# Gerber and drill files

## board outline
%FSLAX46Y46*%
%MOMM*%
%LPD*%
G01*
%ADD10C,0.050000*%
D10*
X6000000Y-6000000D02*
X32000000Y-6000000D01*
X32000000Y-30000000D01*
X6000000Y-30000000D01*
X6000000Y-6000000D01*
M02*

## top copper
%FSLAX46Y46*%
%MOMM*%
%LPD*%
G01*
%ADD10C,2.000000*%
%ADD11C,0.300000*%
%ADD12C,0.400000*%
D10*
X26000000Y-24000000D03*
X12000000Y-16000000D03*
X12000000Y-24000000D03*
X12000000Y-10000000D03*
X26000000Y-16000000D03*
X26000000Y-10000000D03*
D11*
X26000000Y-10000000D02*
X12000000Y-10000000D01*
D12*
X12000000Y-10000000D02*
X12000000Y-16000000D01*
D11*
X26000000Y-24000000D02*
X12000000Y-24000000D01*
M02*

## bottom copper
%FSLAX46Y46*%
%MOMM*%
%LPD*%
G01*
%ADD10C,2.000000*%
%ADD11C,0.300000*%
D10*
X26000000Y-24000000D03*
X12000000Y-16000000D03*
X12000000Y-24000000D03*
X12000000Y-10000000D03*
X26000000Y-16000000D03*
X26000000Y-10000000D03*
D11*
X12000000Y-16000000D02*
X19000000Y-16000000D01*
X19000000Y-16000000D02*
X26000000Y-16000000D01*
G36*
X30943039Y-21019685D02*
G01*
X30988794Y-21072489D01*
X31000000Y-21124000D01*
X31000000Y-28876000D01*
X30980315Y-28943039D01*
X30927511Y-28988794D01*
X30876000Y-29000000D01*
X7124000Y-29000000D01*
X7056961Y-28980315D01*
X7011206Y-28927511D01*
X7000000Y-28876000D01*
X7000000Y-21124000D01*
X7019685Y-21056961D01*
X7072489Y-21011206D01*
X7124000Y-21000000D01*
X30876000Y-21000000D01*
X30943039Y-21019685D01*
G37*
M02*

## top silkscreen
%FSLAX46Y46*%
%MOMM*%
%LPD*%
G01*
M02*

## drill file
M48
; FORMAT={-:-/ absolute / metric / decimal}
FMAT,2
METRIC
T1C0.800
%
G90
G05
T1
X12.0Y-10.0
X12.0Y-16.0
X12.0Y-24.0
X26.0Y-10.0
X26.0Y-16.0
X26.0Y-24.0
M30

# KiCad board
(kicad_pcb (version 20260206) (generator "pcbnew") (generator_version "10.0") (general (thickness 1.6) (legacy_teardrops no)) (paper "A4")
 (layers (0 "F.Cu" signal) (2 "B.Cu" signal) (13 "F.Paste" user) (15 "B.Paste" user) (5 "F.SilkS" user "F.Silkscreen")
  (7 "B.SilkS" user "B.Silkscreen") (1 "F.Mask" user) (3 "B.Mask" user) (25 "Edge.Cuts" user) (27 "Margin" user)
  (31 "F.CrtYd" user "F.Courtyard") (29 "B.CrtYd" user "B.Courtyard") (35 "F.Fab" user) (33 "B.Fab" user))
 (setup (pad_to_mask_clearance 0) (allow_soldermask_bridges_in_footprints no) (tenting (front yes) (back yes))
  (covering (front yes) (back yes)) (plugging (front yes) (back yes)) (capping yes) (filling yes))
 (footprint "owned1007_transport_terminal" (layer "F.Cu") (at 26 24)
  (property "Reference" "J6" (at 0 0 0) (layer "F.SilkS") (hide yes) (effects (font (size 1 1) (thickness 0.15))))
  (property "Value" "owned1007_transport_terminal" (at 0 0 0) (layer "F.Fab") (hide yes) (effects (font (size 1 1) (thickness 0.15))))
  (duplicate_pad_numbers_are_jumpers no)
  (pad "1" thru_hole circle (at 0 0) (size 2 2) (drill 0.8) (layers "*.Cu" "*.Mask") (remove_unused_layers no) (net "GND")))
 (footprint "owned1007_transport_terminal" (layer "F.Cu") (at 12 16)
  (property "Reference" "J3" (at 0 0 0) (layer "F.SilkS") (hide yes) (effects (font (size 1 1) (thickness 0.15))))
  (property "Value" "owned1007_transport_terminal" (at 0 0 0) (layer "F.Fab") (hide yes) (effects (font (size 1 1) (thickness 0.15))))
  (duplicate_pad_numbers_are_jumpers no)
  (pad "1" thru_hole circle (at 0 0) (size 2 2) (drill 0.8) (layers "*.Cu" "*.Mask") (remove_unused_layers no) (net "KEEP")))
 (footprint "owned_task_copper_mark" (layer "F.Cu") (at 10 28)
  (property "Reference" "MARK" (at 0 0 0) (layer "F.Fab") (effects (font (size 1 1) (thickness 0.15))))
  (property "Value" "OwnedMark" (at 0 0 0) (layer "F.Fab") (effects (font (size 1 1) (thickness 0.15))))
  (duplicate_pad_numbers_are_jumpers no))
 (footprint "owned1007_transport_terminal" (layer "F.Cu") (at 12 24)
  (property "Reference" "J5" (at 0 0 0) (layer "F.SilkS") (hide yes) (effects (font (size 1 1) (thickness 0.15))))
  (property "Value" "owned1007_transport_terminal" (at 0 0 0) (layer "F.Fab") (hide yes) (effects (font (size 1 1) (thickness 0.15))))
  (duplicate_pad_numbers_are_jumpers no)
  (pad "1" thru_hole circle (at 0 0) (size 2 2) (drill 0.8) (layers "*.Cu" "*.Mask") (remove_unused_layers no) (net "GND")))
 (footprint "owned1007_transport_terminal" (layer "F.Cu") (at 12 10)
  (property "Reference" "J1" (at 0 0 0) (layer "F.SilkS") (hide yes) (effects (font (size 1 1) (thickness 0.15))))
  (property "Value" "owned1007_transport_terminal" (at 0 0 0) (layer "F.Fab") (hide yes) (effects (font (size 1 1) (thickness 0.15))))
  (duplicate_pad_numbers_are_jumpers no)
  (pad "1" thru_hole circle (at 0 0) (size 2 2) (drill 0.8) (layers "*.Cu" "*.Mask") (remove_unused_layers no) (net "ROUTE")))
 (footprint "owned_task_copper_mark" (layer "F.Cu") (at 13 28)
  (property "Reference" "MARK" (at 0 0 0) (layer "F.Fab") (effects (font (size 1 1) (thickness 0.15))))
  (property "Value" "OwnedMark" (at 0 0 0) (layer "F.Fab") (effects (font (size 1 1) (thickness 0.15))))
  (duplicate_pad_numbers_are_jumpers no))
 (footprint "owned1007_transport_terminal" (layer "F.Cu") (at 26 16)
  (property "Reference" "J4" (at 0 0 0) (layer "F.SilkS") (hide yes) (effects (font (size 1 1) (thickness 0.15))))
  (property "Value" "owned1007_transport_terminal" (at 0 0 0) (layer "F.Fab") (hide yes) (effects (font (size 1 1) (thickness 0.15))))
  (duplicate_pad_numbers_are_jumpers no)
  (pad "1" thru_hole circle (at 0 0) (size 2 2) (drill 0.8) (layers "*.Cu" "*.Mask") (remove_unused_layers no) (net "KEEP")))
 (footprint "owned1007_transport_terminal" (layer "F.Cu") (at 26 10)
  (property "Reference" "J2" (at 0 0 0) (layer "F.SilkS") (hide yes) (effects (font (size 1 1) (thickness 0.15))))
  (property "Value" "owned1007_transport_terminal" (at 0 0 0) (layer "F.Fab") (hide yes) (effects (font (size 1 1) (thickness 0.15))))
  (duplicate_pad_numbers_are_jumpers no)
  (pad "1" thru_hole circle (at 0 0) (size 2 2) (drill 0.8) (layers "*.Cu" "*.Mask") (remove_unused_layers no) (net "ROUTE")))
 (gr_rect (start 6 6) (end 32 30) (stroke (width 0.05) (type default)) (fill no) (layer "Edge.Cuts"))
 (segment (start 26 10) (end 12 10) (width 0.3) (layer "F.Cu") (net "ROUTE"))
 (segment (start 12 10) (end 12 16) (width 0.4) (layer "F.Cu") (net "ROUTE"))
 (segment (start 12 16) (end 19 16) (width 0.3) (locked yes) (layer "B.Cu") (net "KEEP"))
 (segment (start 19 16) (end 26 16) (width 0.3) (layer "B.Cu") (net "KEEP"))
 (segment (start 26 24) (end 12 24) (width 0.3) (layer "F.Cu") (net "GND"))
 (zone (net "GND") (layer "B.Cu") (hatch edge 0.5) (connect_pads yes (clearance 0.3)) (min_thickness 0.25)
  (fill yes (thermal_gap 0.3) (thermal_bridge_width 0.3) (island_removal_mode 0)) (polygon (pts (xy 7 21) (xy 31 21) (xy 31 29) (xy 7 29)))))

